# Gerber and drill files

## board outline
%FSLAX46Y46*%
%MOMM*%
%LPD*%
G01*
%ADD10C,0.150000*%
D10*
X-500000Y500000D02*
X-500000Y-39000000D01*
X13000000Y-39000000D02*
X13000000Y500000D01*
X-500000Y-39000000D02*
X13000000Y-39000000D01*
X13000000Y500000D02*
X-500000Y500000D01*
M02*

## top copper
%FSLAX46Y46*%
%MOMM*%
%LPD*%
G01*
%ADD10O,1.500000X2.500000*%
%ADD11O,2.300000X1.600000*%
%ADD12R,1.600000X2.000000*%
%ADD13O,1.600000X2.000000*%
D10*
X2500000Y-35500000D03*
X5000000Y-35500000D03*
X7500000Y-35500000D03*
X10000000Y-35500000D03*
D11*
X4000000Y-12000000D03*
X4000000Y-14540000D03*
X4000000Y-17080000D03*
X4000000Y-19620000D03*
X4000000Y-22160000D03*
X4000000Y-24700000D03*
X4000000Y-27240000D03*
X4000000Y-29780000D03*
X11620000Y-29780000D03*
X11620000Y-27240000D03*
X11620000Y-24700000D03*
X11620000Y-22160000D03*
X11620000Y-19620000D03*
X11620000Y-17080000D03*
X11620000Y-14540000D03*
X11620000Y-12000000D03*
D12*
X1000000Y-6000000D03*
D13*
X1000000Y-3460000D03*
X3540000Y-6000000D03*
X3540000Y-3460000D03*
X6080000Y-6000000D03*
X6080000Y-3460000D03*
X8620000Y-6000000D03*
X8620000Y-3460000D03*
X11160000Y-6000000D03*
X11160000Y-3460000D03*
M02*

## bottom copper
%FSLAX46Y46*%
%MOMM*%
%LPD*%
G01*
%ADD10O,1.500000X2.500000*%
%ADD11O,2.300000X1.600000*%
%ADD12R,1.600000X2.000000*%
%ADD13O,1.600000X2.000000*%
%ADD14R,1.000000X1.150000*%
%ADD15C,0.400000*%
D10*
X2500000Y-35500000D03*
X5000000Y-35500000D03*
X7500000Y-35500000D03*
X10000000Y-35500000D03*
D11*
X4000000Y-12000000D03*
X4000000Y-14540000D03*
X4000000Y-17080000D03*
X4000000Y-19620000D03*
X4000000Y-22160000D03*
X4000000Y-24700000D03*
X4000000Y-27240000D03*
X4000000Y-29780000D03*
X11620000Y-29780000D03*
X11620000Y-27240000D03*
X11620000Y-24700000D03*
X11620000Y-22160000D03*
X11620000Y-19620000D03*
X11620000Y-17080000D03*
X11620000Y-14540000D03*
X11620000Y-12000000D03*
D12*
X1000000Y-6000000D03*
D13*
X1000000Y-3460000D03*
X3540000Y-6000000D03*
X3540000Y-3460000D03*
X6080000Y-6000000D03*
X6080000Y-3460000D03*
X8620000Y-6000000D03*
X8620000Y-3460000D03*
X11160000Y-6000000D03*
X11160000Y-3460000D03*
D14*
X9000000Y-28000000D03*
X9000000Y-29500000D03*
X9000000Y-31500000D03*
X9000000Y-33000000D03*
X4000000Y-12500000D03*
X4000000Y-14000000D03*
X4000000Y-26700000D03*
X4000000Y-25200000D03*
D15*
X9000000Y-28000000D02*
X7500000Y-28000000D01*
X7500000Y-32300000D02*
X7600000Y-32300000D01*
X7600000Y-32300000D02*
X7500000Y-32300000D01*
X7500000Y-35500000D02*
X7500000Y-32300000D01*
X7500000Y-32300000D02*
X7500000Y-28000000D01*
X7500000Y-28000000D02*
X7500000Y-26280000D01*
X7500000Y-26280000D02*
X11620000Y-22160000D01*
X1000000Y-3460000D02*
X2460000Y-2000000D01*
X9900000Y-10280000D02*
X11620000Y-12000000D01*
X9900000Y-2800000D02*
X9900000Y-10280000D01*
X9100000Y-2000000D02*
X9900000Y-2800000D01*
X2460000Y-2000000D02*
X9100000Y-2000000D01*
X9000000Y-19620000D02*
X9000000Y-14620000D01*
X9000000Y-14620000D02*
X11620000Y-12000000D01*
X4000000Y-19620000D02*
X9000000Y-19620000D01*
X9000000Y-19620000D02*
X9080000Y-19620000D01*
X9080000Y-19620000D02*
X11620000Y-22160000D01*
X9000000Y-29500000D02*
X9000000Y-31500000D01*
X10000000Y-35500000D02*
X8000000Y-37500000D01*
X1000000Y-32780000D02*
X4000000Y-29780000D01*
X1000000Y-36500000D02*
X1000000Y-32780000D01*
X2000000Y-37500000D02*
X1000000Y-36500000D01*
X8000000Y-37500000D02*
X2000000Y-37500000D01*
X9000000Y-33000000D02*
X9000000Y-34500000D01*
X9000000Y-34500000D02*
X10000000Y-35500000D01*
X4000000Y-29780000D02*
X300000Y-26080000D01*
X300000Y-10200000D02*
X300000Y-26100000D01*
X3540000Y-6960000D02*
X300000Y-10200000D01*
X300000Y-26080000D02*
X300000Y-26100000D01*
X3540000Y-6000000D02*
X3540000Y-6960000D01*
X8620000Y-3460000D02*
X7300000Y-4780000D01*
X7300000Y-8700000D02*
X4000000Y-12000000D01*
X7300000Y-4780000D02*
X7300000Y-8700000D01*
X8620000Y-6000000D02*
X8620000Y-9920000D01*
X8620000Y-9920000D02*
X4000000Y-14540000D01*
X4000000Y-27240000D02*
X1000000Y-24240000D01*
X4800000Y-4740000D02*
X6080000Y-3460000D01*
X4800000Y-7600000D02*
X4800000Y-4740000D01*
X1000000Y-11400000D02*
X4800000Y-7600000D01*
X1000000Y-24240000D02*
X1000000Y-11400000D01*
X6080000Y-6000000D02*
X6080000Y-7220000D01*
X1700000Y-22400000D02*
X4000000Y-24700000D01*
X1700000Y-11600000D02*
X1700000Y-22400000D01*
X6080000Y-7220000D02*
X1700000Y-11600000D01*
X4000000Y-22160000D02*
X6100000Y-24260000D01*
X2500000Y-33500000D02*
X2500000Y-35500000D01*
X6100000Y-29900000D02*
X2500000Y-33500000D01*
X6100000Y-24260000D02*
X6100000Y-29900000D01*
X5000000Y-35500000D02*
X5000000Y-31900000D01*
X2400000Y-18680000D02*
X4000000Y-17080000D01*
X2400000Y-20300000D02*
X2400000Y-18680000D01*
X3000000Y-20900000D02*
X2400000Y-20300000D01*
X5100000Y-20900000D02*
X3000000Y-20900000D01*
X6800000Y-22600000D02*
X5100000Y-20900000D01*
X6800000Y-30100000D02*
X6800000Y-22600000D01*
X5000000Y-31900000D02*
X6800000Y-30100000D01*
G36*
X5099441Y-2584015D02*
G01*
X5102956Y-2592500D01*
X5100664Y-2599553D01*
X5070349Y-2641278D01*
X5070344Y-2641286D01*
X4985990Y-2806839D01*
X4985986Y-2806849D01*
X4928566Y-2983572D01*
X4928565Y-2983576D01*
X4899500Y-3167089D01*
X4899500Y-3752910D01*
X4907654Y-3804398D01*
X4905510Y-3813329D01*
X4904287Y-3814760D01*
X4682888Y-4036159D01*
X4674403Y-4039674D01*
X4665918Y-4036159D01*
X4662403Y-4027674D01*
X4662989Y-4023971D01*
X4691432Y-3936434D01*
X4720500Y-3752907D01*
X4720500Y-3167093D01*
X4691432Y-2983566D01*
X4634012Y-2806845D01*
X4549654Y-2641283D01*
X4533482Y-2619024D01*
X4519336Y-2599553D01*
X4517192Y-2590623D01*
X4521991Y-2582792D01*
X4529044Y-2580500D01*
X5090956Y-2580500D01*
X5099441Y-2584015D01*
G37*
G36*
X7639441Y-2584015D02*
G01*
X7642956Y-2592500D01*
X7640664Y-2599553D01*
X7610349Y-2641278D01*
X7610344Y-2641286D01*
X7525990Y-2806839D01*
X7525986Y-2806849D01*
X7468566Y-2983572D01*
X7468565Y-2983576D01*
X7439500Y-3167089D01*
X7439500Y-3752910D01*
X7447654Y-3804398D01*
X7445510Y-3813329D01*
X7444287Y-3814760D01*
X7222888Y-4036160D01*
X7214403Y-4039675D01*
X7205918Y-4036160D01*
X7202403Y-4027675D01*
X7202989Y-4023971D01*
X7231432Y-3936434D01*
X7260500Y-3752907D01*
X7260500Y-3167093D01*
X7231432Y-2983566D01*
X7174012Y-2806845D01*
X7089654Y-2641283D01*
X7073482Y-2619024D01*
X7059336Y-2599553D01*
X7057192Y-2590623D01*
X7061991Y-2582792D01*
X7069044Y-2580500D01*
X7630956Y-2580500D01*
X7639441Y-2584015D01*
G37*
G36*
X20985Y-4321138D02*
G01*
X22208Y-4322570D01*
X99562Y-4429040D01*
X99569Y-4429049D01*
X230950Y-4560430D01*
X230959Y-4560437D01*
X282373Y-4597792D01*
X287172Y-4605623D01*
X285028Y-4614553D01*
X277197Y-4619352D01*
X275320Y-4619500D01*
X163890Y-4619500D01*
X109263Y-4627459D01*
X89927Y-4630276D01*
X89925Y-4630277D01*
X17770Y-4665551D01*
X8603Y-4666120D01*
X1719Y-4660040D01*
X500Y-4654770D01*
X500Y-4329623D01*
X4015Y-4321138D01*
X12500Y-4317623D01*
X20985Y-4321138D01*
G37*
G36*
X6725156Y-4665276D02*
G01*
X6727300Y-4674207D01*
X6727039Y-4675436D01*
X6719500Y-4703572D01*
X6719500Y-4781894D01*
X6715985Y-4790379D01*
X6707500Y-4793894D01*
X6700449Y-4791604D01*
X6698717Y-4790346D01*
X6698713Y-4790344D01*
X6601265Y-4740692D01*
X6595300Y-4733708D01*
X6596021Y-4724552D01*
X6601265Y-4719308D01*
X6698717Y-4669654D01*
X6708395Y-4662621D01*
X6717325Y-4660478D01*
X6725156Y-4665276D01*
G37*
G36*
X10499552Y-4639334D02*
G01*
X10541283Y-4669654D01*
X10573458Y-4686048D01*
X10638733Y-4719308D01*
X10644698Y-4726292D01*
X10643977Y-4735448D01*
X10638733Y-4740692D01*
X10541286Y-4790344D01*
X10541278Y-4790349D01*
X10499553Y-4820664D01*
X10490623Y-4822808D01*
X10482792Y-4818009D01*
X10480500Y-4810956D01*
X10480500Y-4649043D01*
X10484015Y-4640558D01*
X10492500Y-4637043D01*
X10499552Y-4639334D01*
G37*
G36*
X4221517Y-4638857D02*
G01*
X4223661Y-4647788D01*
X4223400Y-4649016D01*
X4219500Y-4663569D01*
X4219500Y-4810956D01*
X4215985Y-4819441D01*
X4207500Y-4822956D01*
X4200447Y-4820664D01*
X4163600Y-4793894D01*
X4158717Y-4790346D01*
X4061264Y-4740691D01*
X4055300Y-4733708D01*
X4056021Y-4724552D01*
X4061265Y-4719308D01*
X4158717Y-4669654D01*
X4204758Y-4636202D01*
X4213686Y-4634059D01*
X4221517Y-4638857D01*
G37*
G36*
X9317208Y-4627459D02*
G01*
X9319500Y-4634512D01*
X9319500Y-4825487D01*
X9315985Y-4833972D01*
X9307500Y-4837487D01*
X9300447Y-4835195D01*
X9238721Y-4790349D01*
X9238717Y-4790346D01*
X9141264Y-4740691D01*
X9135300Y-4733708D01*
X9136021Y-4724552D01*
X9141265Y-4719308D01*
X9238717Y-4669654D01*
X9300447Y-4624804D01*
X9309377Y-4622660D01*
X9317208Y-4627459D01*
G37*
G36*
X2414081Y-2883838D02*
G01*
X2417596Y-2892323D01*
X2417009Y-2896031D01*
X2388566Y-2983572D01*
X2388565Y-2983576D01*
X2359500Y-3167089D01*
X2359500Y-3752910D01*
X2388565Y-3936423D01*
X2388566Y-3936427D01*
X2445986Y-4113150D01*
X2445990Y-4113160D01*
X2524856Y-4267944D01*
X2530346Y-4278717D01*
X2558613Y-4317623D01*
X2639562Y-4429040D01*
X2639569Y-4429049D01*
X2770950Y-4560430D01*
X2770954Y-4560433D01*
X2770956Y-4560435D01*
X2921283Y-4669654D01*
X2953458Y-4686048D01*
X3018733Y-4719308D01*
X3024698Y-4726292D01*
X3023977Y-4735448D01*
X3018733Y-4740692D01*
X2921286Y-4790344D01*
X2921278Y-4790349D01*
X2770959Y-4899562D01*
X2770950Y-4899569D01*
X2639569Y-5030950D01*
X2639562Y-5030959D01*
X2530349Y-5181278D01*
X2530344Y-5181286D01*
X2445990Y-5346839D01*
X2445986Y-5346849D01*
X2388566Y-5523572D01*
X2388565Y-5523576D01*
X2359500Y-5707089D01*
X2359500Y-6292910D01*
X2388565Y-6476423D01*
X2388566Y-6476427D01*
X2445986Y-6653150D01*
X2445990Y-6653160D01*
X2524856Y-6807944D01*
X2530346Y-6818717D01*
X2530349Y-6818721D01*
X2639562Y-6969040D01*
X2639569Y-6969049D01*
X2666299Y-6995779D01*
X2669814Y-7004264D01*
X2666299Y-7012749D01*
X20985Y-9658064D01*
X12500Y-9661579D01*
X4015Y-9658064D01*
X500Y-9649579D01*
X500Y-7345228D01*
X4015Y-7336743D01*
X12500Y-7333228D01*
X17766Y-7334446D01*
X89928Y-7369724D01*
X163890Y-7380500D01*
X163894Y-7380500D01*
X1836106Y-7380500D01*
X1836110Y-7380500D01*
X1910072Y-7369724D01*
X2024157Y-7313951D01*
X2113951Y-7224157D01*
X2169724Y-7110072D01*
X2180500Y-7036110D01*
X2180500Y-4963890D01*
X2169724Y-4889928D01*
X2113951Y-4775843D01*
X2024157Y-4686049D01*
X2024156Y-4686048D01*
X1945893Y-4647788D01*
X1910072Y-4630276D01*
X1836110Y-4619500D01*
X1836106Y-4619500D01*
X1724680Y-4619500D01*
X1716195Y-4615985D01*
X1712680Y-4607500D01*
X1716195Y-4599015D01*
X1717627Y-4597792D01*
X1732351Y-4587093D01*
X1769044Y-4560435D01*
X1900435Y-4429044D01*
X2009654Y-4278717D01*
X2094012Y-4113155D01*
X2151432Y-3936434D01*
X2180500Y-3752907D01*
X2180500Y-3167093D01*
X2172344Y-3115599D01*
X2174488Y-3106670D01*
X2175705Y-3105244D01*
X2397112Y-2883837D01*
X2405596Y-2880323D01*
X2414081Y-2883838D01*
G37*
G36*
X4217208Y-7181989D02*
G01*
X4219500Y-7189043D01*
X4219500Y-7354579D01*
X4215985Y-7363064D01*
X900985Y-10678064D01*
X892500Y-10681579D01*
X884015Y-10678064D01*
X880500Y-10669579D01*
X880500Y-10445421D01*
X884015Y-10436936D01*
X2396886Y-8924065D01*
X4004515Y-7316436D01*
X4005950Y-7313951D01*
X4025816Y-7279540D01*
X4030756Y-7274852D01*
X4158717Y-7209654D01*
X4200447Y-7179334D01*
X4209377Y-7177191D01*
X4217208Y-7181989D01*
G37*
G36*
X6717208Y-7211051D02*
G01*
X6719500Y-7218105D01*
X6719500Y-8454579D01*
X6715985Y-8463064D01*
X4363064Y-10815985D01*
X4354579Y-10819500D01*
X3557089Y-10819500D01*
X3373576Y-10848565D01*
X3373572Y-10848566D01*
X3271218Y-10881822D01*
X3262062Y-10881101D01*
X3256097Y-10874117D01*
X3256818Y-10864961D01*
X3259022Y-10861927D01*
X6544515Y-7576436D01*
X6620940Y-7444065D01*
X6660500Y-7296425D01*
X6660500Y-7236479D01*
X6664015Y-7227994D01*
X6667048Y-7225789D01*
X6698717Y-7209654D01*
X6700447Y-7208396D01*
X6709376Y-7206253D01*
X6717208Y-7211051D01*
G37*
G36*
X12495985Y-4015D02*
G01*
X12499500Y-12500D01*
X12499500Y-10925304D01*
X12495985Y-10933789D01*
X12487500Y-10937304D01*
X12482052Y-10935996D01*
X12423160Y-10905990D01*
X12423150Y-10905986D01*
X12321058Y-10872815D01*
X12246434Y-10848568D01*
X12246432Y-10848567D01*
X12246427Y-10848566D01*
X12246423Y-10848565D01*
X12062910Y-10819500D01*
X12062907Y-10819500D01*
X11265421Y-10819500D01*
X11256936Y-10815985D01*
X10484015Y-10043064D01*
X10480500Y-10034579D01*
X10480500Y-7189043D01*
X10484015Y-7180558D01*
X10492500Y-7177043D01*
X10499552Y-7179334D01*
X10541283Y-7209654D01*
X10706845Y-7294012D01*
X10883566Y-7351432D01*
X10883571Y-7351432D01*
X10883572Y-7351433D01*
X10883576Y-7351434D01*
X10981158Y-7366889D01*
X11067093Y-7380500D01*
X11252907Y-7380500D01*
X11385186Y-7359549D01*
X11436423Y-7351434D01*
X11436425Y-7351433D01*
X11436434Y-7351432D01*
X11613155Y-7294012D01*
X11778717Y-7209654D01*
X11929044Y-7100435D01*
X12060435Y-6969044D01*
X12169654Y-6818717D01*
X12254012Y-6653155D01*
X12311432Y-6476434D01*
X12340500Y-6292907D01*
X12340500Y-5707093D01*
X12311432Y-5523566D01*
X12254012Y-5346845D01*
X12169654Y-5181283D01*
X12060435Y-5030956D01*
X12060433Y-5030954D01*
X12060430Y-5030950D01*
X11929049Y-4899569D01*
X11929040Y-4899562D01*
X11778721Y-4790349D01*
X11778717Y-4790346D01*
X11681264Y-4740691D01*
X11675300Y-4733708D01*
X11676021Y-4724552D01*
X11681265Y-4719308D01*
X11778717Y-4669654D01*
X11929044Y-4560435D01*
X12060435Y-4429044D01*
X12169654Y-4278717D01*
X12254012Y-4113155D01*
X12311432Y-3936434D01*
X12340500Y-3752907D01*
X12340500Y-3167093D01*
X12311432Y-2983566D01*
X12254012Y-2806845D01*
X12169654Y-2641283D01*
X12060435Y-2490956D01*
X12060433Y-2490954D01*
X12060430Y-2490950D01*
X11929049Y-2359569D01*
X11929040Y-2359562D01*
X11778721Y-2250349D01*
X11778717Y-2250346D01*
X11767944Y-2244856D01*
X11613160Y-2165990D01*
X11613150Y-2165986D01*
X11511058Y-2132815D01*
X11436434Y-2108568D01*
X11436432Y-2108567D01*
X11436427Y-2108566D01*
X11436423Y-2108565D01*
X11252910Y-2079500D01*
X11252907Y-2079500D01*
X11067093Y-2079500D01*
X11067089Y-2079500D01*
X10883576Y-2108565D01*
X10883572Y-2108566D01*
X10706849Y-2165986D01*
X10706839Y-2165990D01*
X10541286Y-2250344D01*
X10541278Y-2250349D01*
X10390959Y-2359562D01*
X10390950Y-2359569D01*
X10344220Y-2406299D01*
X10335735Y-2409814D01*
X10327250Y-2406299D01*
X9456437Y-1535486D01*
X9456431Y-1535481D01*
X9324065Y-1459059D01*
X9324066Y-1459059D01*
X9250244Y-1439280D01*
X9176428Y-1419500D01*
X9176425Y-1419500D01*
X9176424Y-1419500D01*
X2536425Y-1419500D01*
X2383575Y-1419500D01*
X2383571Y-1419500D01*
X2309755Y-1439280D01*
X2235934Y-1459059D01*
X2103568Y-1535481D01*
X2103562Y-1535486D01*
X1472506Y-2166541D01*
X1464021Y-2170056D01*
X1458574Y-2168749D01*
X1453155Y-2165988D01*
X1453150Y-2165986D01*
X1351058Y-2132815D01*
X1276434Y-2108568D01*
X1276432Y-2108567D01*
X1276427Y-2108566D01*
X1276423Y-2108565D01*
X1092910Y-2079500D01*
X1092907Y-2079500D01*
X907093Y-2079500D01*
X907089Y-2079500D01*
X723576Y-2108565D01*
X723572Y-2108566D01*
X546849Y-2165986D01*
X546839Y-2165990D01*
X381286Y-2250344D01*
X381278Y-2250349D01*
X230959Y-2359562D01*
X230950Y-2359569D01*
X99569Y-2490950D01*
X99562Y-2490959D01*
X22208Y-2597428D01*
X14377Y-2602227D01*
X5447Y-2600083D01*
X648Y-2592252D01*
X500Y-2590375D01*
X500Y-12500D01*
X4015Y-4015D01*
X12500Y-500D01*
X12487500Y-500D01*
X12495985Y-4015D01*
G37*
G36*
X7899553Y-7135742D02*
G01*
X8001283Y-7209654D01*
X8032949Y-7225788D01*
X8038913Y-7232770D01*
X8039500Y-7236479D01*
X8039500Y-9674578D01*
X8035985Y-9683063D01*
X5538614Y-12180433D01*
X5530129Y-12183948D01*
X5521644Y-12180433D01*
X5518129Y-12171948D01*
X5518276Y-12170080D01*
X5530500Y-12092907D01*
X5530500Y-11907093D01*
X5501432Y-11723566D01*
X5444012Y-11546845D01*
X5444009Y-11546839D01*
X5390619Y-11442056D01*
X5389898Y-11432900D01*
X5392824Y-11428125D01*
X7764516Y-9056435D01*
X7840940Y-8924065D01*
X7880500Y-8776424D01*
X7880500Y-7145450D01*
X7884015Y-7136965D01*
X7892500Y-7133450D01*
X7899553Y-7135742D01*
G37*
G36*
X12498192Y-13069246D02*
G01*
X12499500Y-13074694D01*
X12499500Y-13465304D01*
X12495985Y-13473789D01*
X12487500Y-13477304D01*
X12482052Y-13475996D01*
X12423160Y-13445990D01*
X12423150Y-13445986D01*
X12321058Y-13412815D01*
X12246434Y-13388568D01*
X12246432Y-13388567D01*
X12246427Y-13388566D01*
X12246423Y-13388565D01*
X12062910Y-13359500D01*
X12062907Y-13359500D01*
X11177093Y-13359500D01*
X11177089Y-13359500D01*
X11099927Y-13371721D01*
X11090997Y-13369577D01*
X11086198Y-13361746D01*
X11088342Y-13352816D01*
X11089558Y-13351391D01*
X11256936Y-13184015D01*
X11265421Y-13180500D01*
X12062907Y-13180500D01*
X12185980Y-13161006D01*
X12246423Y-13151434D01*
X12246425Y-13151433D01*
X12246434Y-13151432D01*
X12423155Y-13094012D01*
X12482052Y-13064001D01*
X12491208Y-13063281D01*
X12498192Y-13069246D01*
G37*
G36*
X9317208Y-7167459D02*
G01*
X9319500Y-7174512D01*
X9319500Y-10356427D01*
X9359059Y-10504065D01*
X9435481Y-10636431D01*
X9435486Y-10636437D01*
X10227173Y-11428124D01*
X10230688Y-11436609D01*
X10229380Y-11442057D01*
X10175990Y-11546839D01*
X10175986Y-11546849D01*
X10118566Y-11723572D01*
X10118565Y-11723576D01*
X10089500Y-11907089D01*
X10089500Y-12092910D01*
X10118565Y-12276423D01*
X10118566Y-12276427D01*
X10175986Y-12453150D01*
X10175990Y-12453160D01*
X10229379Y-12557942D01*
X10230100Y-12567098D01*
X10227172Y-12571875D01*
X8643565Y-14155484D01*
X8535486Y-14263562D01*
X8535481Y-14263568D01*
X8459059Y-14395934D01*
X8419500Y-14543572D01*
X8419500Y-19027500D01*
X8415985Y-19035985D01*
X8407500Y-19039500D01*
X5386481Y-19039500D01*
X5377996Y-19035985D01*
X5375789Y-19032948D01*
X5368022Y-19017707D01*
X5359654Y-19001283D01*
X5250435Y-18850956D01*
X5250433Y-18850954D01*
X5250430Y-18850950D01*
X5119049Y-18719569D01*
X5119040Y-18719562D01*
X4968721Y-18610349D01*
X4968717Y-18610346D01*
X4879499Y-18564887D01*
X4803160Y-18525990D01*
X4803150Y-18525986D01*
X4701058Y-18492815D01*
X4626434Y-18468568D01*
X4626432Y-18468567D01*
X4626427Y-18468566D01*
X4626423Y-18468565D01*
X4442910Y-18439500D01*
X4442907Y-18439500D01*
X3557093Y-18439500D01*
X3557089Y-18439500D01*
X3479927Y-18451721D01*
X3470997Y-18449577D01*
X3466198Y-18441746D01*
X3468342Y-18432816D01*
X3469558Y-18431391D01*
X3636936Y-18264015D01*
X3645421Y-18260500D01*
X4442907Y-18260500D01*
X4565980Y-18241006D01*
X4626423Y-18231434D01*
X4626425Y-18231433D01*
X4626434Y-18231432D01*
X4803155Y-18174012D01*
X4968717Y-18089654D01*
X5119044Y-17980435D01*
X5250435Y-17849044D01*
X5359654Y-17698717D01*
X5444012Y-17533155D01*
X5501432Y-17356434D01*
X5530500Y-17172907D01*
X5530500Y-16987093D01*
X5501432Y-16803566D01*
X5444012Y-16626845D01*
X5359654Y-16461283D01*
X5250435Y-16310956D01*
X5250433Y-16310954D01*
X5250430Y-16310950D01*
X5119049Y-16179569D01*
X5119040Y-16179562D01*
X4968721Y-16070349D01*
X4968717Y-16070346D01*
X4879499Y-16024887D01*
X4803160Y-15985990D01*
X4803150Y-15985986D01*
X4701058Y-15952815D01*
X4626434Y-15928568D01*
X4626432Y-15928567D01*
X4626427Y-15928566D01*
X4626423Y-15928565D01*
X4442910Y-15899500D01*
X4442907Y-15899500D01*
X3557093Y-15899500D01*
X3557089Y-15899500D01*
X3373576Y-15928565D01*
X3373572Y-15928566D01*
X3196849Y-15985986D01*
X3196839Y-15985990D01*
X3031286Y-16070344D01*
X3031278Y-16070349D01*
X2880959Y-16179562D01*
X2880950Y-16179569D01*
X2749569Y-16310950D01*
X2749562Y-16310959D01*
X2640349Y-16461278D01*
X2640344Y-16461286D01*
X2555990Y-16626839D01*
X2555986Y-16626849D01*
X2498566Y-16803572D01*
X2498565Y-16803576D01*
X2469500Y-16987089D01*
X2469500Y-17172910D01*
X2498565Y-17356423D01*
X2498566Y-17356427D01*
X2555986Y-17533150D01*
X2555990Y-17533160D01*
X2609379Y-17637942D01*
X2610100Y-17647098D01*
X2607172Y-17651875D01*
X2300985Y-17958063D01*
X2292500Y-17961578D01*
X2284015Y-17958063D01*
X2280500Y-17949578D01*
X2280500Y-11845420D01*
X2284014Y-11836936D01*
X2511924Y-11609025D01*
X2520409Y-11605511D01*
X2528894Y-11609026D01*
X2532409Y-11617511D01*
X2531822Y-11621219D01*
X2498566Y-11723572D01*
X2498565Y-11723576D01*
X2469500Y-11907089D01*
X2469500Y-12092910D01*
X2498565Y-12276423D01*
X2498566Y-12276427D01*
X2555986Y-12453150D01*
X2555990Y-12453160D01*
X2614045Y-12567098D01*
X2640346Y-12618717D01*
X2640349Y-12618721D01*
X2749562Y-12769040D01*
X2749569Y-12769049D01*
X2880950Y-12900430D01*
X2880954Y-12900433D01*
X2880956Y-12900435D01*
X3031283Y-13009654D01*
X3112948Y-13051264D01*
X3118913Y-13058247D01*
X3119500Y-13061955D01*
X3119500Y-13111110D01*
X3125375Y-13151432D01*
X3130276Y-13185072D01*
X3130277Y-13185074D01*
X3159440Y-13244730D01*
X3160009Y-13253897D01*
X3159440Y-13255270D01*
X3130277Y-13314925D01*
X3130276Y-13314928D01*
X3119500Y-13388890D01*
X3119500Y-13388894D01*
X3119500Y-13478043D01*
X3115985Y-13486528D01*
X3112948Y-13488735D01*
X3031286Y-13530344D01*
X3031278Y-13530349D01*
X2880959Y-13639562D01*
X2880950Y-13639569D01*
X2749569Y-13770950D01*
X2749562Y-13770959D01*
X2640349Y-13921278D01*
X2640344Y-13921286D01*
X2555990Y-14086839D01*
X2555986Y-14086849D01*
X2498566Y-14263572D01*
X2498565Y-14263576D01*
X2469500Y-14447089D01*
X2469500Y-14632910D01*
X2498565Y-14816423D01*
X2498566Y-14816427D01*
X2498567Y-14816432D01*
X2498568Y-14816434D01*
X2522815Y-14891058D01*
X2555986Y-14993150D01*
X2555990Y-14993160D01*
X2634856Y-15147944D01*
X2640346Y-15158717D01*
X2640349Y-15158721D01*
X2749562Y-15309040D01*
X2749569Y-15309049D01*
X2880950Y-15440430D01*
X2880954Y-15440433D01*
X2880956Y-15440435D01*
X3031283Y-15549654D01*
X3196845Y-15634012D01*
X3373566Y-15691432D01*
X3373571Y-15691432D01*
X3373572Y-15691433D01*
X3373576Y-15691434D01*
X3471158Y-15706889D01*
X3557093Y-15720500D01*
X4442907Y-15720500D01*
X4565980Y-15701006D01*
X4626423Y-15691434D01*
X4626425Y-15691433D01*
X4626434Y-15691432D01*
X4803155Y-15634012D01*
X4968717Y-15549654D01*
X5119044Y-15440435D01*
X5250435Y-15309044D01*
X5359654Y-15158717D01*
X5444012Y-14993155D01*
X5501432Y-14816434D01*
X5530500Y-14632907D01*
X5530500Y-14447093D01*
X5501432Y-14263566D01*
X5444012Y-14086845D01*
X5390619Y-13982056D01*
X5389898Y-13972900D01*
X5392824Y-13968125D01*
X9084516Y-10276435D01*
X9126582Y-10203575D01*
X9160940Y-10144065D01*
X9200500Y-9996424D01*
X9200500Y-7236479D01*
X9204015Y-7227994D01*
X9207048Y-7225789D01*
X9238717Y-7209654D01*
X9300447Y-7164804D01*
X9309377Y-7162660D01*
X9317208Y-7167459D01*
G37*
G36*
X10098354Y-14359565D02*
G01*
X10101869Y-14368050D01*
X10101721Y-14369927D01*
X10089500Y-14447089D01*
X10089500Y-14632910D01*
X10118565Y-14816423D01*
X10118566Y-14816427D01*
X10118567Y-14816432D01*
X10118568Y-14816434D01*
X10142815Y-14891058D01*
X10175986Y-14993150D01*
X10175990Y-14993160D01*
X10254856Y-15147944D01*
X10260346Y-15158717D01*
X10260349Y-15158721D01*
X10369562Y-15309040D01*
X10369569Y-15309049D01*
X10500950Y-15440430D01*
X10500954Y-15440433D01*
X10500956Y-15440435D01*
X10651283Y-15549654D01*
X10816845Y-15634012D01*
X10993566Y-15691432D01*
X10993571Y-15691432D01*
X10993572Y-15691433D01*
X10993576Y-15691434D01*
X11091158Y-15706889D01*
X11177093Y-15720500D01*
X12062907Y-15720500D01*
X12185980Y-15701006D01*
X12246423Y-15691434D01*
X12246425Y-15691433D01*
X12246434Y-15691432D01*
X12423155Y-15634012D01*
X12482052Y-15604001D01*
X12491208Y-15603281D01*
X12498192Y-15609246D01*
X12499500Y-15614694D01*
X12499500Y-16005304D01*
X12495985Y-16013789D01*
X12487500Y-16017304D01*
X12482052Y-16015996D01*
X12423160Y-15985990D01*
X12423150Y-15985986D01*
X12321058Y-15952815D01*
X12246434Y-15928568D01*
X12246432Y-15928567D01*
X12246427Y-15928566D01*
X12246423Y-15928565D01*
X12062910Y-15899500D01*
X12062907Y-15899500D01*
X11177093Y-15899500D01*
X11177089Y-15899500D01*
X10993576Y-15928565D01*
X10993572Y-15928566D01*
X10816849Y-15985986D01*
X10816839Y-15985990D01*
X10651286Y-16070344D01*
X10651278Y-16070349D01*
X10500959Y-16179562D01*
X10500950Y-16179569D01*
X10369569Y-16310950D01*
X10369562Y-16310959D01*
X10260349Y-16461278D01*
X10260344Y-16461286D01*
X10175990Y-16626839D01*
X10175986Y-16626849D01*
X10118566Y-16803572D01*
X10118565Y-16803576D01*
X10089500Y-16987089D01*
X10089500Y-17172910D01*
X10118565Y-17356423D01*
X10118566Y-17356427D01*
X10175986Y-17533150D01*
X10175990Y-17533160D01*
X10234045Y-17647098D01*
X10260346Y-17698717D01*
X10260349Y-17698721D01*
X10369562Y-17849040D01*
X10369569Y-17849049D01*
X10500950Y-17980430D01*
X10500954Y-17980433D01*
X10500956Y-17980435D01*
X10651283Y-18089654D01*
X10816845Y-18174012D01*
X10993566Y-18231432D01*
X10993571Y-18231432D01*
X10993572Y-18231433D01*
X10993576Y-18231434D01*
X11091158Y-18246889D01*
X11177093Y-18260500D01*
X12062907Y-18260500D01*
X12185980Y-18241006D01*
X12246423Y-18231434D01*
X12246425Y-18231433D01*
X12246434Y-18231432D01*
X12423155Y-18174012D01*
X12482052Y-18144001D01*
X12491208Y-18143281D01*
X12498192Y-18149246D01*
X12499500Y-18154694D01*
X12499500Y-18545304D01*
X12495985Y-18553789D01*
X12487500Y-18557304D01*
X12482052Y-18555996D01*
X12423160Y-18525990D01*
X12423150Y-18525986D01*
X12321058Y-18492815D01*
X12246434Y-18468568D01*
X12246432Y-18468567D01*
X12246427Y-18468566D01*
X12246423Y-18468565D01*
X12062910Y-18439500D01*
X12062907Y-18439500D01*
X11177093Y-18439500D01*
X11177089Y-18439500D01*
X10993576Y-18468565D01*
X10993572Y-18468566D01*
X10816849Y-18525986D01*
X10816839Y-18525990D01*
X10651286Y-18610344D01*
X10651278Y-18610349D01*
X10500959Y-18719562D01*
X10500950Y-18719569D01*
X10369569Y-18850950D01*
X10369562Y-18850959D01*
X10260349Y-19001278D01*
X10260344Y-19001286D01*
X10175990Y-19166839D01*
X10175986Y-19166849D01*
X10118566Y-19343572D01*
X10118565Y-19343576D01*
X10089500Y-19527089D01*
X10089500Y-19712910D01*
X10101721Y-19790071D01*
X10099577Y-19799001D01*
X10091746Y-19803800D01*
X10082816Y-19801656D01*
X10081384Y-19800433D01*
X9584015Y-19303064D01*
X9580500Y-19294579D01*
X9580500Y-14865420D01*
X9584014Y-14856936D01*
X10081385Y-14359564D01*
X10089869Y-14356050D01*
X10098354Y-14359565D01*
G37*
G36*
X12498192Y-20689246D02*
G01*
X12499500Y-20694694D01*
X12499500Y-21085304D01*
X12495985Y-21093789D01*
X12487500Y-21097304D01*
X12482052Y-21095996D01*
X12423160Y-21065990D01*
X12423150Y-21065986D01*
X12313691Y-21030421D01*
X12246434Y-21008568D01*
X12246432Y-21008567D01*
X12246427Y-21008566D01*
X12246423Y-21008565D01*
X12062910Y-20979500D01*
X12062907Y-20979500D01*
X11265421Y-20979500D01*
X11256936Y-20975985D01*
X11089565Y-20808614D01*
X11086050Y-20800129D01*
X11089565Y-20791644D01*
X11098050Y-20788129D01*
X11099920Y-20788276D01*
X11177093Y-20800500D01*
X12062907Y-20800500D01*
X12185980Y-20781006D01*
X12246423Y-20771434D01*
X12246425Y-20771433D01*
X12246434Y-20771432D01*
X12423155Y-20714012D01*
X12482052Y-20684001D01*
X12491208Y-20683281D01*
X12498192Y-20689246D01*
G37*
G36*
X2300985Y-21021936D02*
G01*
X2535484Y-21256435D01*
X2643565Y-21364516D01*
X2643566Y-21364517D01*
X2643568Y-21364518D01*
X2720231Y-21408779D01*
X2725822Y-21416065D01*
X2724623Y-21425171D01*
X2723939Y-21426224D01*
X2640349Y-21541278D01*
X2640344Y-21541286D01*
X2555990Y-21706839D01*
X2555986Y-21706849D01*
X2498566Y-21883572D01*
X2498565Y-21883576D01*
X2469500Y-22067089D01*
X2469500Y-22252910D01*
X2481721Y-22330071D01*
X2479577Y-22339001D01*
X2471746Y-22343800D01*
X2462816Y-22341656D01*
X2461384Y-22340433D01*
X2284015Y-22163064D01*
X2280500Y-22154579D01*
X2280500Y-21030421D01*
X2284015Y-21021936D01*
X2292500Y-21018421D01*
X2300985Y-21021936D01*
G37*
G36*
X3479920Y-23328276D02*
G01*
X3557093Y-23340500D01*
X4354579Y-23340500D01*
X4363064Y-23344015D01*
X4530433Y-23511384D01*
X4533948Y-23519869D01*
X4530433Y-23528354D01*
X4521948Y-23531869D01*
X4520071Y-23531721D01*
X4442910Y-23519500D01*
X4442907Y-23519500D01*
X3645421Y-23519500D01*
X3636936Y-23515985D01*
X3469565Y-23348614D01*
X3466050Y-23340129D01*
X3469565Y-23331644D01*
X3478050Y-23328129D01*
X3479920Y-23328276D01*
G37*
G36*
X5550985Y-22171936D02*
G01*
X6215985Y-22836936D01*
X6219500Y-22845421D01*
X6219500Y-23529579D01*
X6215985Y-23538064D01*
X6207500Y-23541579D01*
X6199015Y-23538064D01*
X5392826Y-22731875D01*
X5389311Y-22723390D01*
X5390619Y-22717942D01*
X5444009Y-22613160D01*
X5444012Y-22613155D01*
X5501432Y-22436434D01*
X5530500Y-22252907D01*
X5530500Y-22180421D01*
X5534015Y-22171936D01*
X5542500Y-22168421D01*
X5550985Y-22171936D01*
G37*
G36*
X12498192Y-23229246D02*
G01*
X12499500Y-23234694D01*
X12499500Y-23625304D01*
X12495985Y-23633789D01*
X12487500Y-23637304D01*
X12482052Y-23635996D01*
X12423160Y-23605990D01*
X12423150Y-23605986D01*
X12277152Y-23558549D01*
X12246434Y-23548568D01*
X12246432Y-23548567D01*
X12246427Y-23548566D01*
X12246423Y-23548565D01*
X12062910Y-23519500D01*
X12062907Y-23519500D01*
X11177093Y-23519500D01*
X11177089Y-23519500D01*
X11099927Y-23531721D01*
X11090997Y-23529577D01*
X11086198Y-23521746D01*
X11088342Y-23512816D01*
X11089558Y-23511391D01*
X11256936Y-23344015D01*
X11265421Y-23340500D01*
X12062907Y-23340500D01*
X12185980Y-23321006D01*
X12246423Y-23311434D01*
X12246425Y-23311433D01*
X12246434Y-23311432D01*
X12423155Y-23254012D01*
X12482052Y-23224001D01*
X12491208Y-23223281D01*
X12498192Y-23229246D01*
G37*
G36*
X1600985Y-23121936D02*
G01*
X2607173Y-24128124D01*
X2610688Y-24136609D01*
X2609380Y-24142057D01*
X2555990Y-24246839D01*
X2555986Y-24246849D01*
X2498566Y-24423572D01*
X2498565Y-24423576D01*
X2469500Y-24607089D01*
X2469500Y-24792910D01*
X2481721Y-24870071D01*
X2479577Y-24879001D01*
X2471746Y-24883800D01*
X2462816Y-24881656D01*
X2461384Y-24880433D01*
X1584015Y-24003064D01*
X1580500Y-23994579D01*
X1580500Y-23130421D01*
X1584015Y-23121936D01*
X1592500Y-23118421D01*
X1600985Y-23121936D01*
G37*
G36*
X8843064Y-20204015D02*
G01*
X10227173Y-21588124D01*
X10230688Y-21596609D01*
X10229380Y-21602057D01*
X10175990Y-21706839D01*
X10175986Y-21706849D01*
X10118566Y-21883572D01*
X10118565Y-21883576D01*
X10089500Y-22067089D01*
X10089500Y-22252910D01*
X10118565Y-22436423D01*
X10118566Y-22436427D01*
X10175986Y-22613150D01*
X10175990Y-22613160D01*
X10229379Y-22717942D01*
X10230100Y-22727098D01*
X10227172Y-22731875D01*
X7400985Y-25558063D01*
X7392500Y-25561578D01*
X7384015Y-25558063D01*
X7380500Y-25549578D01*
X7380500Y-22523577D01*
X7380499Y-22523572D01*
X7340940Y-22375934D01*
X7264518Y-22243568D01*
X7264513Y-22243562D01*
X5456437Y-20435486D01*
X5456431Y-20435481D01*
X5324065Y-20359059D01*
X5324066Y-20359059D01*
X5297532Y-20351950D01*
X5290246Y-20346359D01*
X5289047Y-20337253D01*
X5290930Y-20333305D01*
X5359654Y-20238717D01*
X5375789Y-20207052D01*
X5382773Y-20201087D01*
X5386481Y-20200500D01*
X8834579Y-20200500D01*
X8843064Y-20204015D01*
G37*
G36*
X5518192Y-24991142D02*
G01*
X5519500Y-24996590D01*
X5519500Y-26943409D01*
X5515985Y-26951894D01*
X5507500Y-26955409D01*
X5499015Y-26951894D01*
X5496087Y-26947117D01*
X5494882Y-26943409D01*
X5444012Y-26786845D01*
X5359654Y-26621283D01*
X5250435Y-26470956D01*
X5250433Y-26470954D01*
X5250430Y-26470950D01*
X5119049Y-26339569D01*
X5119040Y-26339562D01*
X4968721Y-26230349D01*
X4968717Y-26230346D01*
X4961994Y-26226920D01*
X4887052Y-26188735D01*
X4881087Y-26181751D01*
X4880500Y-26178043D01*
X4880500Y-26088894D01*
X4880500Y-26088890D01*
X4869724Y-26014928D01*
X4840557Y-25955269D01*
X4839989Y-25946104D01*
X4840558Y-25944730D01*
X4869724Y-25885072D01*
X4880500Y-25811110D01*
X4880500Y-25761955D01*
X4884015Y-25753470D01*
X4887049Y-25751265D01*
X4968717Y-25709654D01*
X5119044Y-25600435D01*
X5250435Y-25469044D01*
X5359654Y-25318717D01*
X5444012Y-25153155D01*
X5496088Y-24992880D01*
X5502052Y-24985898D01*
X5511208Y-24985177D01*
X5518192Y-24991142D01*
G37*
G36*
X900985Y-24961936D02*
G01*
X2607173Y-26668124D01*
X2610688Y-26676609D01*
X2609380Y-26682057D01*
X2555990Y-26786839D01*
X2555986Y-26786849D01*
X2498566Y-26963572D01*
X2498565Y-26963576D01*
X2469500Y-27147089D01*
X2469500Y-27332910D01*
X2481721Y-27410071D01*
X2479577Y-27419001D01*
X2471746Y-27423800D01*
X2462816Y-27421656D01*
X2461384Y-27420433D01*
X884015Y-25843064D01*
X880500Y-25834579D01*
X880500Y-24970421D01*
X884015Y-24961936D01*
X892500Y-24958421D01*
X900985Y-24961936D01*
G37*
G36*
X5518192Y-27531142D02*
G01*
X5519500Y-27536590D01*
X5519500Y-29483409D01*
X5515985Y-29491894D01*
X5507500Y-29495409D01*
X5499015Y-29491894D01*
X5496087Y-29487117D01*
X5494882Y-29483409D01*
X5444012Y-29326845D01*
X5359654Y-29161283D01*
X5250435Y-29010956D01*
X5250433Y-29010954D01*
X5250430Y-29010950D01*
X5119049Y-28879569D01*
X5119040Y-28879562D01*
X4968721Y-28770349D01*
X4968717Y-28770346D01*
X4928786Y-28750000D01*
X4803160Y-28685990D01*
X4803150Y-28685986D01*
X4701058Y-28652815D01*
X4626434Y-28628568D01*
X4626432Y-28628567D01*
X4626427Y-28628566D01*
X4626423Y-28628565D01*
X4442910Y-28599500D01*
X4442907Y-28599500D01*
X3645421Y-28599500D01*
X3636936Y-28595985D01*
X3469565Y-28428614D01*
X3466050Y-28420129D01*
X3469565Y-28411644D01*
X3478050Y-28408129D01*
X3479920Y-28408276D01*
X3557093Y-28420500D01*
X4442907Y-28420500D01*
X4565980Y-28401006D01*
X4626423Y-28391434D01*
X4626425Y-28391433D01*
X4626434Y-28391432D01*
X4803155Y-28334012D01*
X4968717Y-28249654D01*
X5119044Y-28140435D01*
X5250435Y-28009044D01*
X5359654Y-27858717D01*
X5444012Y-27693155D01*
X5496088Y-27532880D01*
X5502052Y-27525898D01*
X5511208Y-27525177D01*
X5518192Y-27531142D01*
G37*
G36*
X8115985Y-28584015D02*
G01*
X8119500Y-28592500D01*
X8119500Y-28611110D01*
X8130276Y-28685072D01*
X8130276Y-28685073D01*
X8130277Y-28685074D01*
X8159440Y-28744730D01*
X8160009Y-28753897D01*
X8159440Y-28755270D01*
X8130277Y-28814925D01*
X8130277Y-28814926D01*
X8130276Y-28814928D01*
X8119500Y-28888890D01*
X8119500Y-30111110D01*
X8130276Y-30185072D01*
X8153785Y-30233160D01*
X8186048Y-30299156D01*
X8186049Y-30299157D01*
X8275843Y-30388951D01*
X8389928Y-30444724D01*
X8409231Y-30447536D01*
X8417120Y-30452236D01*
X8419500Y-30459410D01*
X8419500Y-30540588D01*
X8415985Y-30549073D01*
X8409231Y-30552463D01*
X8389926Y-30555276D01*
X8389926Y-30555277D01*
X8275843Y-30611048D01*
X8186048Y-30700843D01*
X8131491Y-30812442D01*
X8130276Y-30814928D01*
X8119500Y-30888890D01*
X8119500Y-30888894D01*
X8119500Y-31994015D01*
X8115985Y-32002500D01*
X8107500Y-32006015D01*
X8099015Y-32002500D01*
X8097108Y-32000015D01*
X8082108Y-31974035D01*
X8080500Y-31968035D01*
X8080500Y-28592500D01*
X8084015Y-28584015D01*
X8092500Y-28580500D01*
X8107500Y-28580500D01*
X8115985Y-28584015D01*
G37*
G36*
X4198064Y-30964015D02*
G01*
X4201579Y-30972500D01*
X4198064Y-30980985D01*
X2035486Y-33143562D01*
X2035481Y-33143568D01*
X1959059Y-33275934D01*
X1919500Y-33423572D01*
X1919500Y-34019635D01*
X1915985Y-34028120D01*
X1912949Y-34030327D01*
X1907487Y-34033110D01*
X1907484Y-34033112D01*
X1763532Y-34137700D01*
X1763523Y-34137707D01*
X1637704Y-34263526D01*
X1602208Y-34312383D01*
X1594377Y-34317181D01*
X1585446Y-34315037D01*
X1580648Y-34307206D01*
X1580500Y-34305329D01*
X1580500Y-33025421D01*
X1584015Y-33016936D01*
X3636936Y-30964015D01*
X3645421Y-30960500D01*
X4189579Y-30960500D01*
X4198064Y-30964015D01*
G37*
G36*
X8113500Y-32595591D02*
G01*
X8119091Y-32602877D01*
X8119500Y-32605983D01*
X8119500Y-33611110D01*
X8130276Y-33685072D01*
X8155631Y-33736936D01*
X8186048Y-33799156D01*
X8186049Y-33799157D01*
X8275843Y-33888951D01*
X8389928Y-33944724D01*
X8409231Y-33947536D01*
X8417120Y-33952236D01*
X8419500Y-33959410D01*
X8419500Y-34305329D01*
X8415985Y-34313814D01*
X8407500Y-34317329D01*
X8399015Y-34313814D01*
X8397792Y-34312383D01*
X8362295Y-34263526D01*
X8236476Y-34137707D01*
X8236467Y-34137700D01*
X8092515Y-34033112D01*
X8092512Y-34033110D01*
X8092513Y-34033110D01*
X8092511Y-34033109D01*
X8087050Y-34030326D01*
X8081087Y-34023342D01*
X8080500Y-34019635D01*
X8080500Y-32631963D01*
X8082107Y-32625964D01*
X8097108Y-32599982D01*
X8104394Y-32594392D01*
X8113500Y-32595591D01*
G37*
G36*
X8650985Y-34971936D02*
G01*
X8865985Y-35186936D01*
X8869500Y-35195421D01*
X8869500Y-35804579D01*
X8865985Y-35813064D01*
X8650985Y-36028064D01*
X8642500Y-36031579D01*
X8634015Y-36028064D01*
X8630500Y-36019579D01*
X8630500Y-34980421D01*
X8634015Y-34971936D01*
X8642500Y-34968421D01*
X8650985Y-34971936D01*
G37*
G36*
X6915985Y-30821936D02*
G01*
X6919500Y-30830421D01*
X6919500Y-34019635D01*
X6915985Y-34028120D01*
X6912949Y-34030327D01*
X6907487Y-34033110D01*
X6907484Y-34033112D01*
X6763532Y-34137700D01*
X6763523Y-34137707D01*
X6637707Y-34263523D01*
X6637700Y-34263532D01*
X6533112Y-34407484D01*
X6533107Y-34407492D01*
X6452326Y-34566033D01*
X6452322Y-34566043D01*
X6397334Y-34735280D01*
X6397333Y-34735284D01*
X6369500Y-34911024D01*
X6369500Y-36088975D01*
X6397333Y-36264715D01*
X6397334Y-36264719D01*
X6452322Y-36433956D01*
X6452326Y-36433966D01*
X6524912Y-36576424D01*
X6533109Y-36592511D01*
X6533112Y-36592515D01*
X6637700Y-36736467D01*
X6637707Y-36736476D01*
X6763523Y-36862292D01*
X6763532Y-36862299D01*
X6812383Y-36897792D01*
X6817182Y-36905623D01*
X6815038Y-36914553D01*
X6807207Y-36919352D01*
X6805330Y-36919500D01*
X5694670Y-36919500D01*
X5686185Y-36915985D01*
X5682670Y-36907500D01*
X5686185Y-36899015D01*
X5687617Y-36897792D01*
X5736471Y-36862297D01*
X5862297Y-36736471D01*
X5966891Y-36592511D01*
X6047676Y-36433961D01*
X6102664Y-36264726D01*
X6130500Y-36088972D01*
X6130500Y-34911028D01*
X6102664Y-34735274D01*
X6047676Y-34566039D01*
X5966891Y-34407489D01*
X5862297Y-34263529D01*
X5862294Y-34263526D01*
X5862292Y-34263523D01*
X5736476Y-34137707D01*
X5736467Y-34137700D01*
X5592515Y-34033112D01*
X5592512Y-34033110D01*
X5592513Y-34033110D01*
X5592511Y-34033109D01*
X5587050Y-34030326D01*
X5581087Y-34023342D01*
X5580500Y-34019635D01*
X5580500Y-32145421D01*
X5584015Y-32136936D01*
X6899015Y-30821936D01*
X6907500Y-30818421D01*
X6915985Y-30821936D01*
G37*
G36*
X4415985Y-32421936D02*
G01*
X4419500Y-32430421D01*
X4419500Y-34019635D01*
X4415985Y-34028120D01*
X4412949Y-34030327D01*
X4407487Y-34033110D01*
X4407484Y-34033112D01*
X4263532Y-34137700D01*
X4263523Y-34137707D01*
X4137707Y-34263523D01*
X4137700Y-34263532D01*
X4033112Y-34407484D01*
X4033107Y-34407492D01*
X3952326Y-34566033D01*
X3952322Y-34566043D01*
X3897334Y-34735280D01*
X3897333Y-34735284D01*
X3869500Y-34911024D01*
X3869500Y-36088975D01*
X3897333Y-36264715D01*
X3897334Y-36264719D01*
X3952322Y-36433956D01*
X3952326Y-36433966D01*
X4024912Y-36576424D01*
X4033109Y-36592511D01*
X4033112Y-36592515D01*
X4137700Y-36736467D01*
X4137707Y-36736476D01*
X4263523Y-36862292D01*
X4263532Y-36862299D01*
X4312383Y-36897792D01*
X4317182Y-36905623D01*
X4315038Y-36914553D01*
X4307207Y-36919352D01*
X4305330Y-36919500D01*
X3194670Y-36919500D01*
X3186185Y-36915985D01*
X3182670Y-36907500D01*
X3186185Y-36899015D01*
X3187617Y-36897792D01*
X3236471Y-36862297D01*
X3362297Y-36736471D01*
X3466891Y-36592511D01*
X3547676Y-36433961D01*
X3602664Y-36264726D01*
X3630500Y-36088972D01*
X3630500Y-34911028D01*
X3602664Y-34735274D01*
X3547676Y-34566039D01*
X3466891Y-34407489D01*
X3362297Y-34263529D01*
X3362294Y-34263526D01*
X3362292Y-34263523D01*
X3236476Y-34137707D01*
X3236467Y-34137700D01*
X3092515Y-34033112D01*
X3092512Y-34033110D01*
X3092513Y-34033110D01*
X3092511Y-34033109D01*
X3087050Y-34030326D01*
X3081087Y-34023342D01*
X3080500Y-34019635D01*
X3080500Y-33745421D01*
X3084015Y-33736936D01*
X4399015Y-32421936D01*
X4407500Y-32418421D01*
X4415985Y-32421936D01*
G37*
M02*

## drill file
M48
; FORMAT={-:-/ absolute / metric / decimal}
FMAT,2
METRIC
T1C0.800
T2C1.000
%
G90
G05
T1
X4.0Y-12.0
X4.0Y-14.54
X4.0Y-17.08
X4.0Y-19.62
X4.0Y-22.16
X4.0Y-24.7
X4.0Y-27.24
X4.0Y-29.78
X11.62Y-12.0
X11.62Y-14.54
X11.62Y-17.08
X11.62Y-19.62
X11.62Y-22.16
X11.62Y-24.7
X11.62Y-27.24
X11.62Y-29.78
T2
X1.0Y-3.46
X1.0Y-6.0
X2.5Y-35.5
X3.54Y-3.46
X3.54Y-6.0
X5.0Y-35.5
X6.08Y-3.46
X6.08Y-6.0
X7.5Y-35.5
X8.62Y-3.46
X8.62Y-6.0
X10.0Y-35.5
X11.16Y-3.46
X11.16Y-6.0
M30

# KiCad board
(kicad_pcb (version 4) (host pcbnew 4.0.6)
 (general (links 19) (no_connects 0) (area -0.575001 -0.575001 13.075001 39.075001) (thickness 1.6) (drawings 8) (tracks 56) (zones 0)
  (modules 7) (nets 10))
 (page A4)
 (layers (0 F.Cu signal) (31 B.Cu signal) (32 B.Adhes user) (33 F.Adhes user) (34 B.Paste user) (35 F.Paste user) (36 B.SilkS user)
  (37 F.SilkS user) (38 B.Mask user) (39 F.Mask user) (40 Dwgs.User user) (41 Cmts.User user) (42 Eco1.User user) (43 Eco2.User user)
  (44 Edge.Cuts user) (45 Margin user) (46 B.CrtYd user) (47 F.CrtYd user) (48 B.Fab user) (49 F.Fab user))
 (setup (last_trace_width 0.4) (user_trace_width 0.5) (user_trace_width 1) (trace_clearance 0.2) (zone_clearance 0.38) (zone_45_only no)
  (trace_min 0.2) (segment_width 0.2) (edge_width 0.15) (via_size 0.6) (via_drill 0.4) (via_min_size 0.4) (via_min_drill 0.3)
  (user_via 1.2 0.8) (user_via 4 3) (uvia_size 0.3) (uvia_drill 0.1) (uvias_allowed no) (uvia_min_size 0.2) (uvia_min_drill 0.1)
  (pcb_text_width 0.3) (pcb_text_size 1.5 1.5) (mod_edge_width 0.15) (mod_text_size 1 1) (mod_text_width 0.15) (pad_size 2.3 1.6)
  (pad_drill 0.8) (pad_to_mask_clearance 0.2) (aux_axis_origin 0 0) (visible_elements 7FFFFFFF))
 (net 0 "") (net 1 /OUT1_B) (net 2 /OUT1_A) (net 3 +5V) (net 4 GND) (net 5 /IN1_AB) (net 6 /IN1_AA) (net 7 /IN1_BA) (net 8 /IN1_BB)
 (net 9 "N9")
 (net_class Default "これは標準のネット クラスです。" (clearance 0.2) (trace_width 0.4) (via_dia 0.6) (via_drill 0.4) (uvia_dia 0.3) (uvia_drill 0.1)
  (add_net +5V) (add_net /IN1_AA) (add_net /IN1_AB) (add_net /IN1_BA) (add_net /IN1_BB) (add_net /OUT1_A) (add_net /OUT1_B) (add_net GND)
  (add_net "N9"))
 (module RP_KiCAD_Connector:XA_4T (layer F.Cu) (at 2.5 35.5)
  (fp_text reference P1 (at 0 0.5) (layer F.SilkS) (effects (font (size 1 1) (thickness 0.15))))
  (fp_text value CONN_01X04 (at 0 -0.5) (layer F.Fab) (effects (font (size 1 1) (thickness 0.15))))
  (pad 4 thru_hole oval (at 0 0) (size 1.5 2.5) (drill 1) (layers *.Cu *.Mask F.SilkS) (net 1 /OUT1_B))
  (pad 3 thru_hole oval (at 2.5 0) (size 1.5 2.5) (drill 1) (layers *.Cu *.Mask F.SilkS) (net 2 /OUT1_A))
  (pad 2 thru_hole oval (at 5 0) (size 1.5 2.5) (drill 1) (layers *.Cu *.Mask F.SilkS) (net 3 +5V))
  (pad 1 thru_hole oval (at 7.5 0) (size 1.5 2.5) (drill 1) (layers *.Cu *.Mask F.SilkS) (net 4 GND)))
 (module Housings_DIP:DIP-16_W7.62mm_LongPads (layer F.Cu) (at 4 12)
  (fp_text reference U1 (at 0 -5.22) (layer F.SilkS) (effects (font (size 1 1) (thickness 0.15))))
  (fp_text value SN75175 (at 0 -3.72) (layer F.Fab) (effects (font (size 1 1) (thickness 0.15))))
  (pad 1 thru_hole oval (at 0 0) (size 2.3 1.6) (drill 0.8) (layers *.Cu *.Mask F.SilkS) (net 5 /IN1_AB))
  (pad 2 thru_hole oval (at 0 2.54) (size 2.3 1.6) (drill 0.8) (layers *.Cu *.Mask F.SilkS) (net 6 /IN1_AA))
  (pad 3 thru_hole oval (at 0 5.08) (size 2.3 1.6) (drill 0.8) (layers *.Cu *.Mask F.SilkS) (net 2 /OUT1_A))
  (pad 4 thru_hole oval (at 0 7.62) (size 2.3 1.6) (drill 0.8) (layers *.Cu *.Mask F.SilkS) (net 3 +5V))
  (pad 5 thru_hole oval (at 0 10.16) (size 2.3 1.6) (drill 0.8) (layers *.Cu *.Mask F.SilkS) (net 1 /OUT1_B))
  (pad 6 thru_hole oval (at 0 12.7) (size 2.3 1.6) (drill 0.8) (layers *.Cu *.Mask F.SilkS) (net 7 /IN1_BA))
  (pad 7 thru_hole oval (at 0 15.24) (size 2.3 1.6) (drill 0.8) (layers *.Cu *.Mask F.SilkS) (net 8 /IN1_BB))
  (pad 8 thru_hole oval (at 0 17.78) (size 2.3 1.6) (drill 0.8) (layers *.Cu *.Mask F.SilkS) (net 4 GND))
  (pad 9 thru_hole oval (at 7.62 17.78) (size 2.3 1.6) (drill 0.8) (layers *.Cu *.Mask F.SilkS))
  (pad 10 thru_hole oval (at 7.62 15.24) (size 2.3 1.6) (drill 0.8) (layers *.Cu *.Mask F.SilkS))
  (pad 11 thru_hole oval (at 7.62 12.7) (size 2.3 1.6) (drill 0.8) (layers *.Cu *.Mask F.SilkS))
  (pad 12 thru_hole oval (at 7.62 10.16) (size 2.3 1.6) (drill 0.8) (layers *.Cu *.Mask F.SilkS) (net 3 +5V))
  (pad 13 thru_hole oval (at 7.62 7.62) (size 2.3 1.6) (drill 0.8) (layers *.Cu *.Mask F.SilkS))
  (pad 14 thru_hole oval (at 7.62 5.08) (size 2.3 1.6) (drill 0.8) (layers *.Cu *.Mask F.SilkS))
  (pad 15 thru_hole oval (at 7.62 2.54) (size 2.3 1.6) (drill 0.8) (layers *.Cu *.Mask F.SilkS))
  (pad 16 thru_hole oval (at 7.62 0) (size 2.3 1.6) (drill 0.8) (layers *.Cu *.Mask F.SilkS) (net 3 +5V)))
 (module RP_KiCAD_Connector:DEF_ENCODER (layer F.Cu) (at 1 6)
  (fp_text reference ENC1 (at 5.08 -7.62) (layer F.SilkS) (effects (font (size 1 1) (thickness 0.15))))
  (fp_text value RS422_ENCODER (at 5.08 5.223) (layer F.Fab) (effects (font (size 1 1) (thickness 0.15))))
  (pad 1 thru_hole rect (at 0 0) (size 1.6 2) (drill 1) (layers *.Cu *.Mask F.SilkS))
  (pad 2 thru_hole oval (at 0 -2.54) (size 1.6 2) (drill 1) (layers *.Cu *.Mask F.SilkS) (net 3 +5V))
  (pad 3 thru_hole oval (at 2.54 0) (size 1.6 2) (drill 1) (layers *.Cu *.Mask F.SilkS) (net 4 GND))
  (pad 4 thru_hole oval (at 2.54 -2.54) (size 1.6 2) (drill 1) (layers *.Cu *.Mask F.SilkS))
  (pad 5 thru_hole oval (at 5.08 0) (size 1.6 2) (drill 1) (layers *.Cu *.Mask F.SilkS) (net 7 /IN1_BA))
  (pad 6 thru_hole oval (at 5.08 -2.54) (size 1.6 2) (drill 1) (layers *.Cu *.Mask F.SilkS) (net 8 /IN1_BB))
  (pad 7 thru_hole oval (at 7.62 0) (size 1.6 2) (drill 1) (layers *.Cu *.Mask F.SilkS) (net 6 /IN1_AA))
  (pad 8 thru_hole oval (at 7.62 -2.54) (size 1.6 2) (drill 1) (layers *.Cu *.Mask F.SilkS) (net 5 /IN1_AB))
  (pad 9 thru_hole oval (at 10.16 0) (size 1.6 2) (drill 1) (layers *.Cu *.Mask F.SilkS))
  (pad 10 thru_hole oval (at 10.16 -2.54) (size 1.6 2) (drill 1) (layers *.Cu *.Mask F.SilkS)))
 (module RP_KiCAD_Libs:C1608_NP (layer B.Cu) (at 9 29 270)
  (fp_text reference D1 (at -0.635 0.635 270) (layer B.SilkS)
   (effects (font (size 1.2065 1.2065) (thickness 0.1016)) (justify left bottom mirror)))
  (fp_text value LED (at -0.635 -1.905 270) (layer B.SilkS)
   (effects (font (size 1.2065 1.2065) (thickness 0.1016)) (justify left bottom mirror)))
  (pad 1 smd rect (at -1 0 270) (size 1.15 1) (layers B.Cu B.Paste B.Mask) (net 3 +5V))
  (pad 2 smd rect (at 0.5 0 270) (size 1.15 1) (layers B.Cu B.Paste B.Mask) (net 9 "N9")))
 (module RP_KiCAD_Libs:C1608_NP (layer B.Cu) (at 9 32.5 270)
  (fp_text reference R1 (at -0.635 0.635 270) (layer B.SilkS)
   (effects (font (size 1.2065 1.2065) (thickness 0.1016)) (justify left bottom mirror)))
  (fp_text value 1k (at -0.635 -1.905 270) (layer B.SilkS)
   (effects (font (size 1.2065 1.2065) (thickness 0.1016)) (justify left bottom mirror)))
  (pad 1 smd rect (at -1 0 270) (size 1.15 1) (layers B.Cu B.Paste B.Mask) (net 9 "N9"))
  (pad 2 smd rect (at 0.5 0 270) (size 1.15 1) (layers B.Cu B.Paste B.Mask) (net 4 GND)))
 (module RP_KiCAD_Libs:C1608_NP (layer B.Cu) (at 4 13.5 270)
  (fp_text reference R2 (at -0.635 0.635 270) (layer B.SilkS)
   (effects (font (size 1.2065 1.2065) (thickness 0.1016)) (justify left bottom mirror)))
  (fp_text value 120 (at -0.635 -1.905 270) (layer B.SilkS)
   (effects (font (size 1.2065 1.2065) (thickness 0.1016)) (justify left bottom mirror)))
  (pad 1 smd rect (at -1 0 270) (size 1.15 1) (layers B.Cu B.Paste B.Mask) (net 5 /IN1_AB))
  (pad 2 smd rect (at 0.5 0 270) (size 1.15 1) (layers B.Cu B.Paste B.Mask) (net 6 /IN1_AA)))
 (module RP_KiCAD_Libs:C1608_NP (layer B.Cu) (at 4 25.7 90)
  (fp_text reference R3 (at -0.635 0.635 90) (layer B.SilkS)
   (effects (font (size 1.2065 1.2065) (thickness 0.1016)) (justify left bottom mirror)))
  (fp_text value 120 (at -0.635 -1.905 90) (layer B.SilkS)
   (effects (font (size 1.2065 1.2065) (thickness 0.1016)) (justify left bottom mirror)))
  (pad 1 smd rect (at -1 0 90) (size 1.15 1) (layers B.Cu B.Paste B.Mask) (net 8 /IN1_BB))
  (pad 2 smd rect (at 0.5 0 90) (size 1.15 1) (layers B.Cu B.Paste B.Mask) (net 7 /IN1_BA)))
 (gr_line (start -0.5 -0.5) (end -0.5 39) (angle 90) (layer Edge.Cuts) (width 0.15))
 (gr_line (start 13 39) (end 13 -0.5) (angle 90) (layer Edge.Cuts) (width 0.15))
 (gr_line (start -0.5 39) (end 13 39) (angle 90) (layer Edge.Cuts) (width 0.15))
 (gr_line (start 13 -0.5) (end -0.5 -0.5) (angle 90) (layer Edge.Cuts) (width 0.15))
 (segment (start 9 28) (end 7.5 28) (width 0.4) (layer B.Cu) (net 3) (status 400000))
 (segment (start 7.5 32.3) (end 7.6 32.3) (width 0.4) (layer B.Cu) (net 3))
 (segment (start 7.6 32.3) (end 7.5 32.3) (width 0.4) (layer B.Cu) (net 3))
 (segment (start 7.5 35.5) (end 7.5 32.3) (width 0.4) (layer B.Cu) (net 3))
 (segment (start 7.5 32.3) (end 7.5 28) (width 0.4) (layer B.Cu) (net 3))
 (segment (start 7.5 28) (end 7.5 26.28) (width 0.4) (layer B.Cu) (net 3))
 (segment (start 7.5 26.28) (end 11.62 22.16) (width 0.4) (layer B.Cu) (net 3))
 (segment (start 1 3.46) (end 2.46 2) (width 0.4) (layer B.Cu) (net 3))
 (segment (start 9.9 10.28) (end 11.62 12) (width 0.4) (layer B.Cu) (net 3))
 (segment (start 9.9 2.8) (end 9.9 10.28) (width 0.4) (layer B.Cu) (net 3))
 (segment (start 9.1 2) (end 9.9 2.8) (width 0.4) (layer B.Cu) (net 3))
 (segment (start 2.46 2) (end 9.1 2) (width 0.4) (layer B.Cu) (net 3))
 (segment (start 9 19.62) (end 9 14.62) (width 0.4) (layer B.Cu) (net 3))
 (segment (start 9 14.62) (end 11.62 12) (width 0.4) (layer B.Cu) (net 3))
 (segment (start 4 19.62) (end 9 19.62) (width 0.4) (layer B.Cu) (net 3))
 (segment (start 9 19.62) (end 9.08 19.62) (width 0.4) (layer B.Cu) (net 3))
 (segment (start 9.08 19.62) (end 11.62 22.16) (width 0.4) (layer B.Cu) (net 3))
 (segment (start 9 29.5) (end 9 31.5) (width 0.4) (layer B.Cu) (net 9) (status C00000))
 (segment (start 10 35.5) (end 8 37.5) (width 0.4) (layer B.Cu) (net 4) (status 400000))
 (segment (start 1 32.78) (end 4 29.78) (width 0.4) (layer B.Cu) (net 4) (status 800000))
 (segment (start 1 36.5) (end 1 32.78) (width 0.4) (layer B.Cu) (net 4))
 (segment (start 2 37.5) (end 1 36.5) (width 0.4) (layer B.Cu) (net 4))
 (segment (start 8 37.5) (end 2 37.5) (width 0.4) (layer B.Cu) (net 4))
 (segment (start 9 33) (end 9 34.5) (width 0.4) (layer B.Cu) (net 4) (status 400000))
 (segment (start 9 34.5) (end 10 35.5) (width 0.4) (layer B.Cu) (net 4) (status 800000))
 (segment (start 4 29.78) (end 0.3 26.08) (width 0.4) (layer B.Cu) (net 4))
 (segment (start 0.3 10.2) (end 0.3 26.1) (width 0.4) (layer B.Cu) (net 4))
 (segment (start 3.54 6.96) (end 0.3 10.2) (width 0.4) (layer B.Cu) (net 4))
 (segment (start 0.3 26.08) (end 0.3 26.1) (width 0.4) (layer B.Cu) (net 4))
 (segment (start 3.54 6) (end 3.54 6.96) (width 0.4) (layer B.Cu) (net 4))
 (segment (start 8.62 3.46) (end 7.3 4.78) (width 0.4) (layer B.Cu) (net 5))
 (segment (start 7.3 8.7) (end 4 12) (width 0.4) (layer B.Cu) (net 5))
 (segment (start 7.3 4.78) (end 7.3 8.7) (width 0.4) (layer B.Cu) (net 5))
 (segment (start 8.62 6) (end 8.62 9.92) (width 0.4) (layer B.Cu) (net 6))
 (segment (start 8.62 9.92) (end 4 14.54) (width 0.4) (layer B.Cu) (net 6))
 (segment (start 4 27.24) (end 1 24.24) (width 0.4) (layer B.Cu) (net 8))
 (segment (start 4.8 4.74) (end 6.08 3.46) (width 0.4) (layer B.Cu) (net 8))
 (segment (start 4.8 7.6) (end 4.8 4.74) (width 0.4) (layer B.Cu) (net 8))
 (segment (start 1 11.4) (end 4.8 7.6) (width 0.4) (layer B.Cu) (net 8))
 (segment (start 1 24.24) (end 1 11.4) (width 0.4) (layer B.Cu) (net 8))
 (segment (start 6.08 6) (end 6.08 7.22) (width 0.4) (layer B.Cu) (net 7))
 (segment (start 1.7 22.4) (end 4 24.7) (width 0.4) (layer B.Cu) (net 7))
 (segment (start 1.7 11.6) (end 1.7 22.4) (width 0.4) (layer B.Cu) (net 7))
 (segment (start 6.08 7.22) (end 1.7 11.6) (width 0.4) (layer B.Cu) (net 7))
 (segment (start 4 22.16) (end 6.1 24.26) (width 0.4) (layer B.Cu) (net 1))
 (segment (start 2.5 33.5) (end 2.5 35.5) (width 0.4) (layer B.Cu) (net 1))
 (segment (start 6.1 29.9) (end 2.5 33.5) (width 0.4) (layer B.Cu) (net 1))
 (segment (start 6.1 24.26) (end 6.1 29.9) (width 0.4) (layer B.Cu) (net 1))
 (segment (start 5 35.5) (end 5 31.9) (width 0.4) (layer B.Cu) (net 2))
 (segment (start 2.4 18.68) (end 4 17.08) (width 0.4) (layer B.Cu) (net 2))
 (segment (start 2.4 20.3) (end 2.4 18.68) (width 0.4) (layer B.Cu) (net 2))
 (segment (start 3 20.9) (end 2.4 20.3) (width 0.4) (layer B.Cu) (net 2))
 (segment (start 5.1 20.9) (end 3 20.9) (width 0.4) (layer B.Cu) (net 2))
 (segment (start 6.8 22.6) (end 5.1 20.9) (width 0.4) (layer B.Cu) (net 2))
 (segment (start 6.8 30.1) (end 6.8 22.6) (width 0.4) (layer B.Cu) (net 2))
 (segment (start 5 31.9) (end 6.8 30.1) (width 0.4) (layer B.Cu) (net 2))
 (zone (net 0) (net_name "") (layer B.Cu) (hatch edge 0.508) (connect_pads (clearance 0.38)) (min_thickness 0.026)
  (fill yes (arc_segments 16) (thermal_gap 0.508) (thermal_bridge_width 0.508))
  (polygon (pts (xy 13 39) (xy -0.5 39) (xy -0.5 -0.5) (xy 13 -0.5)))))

